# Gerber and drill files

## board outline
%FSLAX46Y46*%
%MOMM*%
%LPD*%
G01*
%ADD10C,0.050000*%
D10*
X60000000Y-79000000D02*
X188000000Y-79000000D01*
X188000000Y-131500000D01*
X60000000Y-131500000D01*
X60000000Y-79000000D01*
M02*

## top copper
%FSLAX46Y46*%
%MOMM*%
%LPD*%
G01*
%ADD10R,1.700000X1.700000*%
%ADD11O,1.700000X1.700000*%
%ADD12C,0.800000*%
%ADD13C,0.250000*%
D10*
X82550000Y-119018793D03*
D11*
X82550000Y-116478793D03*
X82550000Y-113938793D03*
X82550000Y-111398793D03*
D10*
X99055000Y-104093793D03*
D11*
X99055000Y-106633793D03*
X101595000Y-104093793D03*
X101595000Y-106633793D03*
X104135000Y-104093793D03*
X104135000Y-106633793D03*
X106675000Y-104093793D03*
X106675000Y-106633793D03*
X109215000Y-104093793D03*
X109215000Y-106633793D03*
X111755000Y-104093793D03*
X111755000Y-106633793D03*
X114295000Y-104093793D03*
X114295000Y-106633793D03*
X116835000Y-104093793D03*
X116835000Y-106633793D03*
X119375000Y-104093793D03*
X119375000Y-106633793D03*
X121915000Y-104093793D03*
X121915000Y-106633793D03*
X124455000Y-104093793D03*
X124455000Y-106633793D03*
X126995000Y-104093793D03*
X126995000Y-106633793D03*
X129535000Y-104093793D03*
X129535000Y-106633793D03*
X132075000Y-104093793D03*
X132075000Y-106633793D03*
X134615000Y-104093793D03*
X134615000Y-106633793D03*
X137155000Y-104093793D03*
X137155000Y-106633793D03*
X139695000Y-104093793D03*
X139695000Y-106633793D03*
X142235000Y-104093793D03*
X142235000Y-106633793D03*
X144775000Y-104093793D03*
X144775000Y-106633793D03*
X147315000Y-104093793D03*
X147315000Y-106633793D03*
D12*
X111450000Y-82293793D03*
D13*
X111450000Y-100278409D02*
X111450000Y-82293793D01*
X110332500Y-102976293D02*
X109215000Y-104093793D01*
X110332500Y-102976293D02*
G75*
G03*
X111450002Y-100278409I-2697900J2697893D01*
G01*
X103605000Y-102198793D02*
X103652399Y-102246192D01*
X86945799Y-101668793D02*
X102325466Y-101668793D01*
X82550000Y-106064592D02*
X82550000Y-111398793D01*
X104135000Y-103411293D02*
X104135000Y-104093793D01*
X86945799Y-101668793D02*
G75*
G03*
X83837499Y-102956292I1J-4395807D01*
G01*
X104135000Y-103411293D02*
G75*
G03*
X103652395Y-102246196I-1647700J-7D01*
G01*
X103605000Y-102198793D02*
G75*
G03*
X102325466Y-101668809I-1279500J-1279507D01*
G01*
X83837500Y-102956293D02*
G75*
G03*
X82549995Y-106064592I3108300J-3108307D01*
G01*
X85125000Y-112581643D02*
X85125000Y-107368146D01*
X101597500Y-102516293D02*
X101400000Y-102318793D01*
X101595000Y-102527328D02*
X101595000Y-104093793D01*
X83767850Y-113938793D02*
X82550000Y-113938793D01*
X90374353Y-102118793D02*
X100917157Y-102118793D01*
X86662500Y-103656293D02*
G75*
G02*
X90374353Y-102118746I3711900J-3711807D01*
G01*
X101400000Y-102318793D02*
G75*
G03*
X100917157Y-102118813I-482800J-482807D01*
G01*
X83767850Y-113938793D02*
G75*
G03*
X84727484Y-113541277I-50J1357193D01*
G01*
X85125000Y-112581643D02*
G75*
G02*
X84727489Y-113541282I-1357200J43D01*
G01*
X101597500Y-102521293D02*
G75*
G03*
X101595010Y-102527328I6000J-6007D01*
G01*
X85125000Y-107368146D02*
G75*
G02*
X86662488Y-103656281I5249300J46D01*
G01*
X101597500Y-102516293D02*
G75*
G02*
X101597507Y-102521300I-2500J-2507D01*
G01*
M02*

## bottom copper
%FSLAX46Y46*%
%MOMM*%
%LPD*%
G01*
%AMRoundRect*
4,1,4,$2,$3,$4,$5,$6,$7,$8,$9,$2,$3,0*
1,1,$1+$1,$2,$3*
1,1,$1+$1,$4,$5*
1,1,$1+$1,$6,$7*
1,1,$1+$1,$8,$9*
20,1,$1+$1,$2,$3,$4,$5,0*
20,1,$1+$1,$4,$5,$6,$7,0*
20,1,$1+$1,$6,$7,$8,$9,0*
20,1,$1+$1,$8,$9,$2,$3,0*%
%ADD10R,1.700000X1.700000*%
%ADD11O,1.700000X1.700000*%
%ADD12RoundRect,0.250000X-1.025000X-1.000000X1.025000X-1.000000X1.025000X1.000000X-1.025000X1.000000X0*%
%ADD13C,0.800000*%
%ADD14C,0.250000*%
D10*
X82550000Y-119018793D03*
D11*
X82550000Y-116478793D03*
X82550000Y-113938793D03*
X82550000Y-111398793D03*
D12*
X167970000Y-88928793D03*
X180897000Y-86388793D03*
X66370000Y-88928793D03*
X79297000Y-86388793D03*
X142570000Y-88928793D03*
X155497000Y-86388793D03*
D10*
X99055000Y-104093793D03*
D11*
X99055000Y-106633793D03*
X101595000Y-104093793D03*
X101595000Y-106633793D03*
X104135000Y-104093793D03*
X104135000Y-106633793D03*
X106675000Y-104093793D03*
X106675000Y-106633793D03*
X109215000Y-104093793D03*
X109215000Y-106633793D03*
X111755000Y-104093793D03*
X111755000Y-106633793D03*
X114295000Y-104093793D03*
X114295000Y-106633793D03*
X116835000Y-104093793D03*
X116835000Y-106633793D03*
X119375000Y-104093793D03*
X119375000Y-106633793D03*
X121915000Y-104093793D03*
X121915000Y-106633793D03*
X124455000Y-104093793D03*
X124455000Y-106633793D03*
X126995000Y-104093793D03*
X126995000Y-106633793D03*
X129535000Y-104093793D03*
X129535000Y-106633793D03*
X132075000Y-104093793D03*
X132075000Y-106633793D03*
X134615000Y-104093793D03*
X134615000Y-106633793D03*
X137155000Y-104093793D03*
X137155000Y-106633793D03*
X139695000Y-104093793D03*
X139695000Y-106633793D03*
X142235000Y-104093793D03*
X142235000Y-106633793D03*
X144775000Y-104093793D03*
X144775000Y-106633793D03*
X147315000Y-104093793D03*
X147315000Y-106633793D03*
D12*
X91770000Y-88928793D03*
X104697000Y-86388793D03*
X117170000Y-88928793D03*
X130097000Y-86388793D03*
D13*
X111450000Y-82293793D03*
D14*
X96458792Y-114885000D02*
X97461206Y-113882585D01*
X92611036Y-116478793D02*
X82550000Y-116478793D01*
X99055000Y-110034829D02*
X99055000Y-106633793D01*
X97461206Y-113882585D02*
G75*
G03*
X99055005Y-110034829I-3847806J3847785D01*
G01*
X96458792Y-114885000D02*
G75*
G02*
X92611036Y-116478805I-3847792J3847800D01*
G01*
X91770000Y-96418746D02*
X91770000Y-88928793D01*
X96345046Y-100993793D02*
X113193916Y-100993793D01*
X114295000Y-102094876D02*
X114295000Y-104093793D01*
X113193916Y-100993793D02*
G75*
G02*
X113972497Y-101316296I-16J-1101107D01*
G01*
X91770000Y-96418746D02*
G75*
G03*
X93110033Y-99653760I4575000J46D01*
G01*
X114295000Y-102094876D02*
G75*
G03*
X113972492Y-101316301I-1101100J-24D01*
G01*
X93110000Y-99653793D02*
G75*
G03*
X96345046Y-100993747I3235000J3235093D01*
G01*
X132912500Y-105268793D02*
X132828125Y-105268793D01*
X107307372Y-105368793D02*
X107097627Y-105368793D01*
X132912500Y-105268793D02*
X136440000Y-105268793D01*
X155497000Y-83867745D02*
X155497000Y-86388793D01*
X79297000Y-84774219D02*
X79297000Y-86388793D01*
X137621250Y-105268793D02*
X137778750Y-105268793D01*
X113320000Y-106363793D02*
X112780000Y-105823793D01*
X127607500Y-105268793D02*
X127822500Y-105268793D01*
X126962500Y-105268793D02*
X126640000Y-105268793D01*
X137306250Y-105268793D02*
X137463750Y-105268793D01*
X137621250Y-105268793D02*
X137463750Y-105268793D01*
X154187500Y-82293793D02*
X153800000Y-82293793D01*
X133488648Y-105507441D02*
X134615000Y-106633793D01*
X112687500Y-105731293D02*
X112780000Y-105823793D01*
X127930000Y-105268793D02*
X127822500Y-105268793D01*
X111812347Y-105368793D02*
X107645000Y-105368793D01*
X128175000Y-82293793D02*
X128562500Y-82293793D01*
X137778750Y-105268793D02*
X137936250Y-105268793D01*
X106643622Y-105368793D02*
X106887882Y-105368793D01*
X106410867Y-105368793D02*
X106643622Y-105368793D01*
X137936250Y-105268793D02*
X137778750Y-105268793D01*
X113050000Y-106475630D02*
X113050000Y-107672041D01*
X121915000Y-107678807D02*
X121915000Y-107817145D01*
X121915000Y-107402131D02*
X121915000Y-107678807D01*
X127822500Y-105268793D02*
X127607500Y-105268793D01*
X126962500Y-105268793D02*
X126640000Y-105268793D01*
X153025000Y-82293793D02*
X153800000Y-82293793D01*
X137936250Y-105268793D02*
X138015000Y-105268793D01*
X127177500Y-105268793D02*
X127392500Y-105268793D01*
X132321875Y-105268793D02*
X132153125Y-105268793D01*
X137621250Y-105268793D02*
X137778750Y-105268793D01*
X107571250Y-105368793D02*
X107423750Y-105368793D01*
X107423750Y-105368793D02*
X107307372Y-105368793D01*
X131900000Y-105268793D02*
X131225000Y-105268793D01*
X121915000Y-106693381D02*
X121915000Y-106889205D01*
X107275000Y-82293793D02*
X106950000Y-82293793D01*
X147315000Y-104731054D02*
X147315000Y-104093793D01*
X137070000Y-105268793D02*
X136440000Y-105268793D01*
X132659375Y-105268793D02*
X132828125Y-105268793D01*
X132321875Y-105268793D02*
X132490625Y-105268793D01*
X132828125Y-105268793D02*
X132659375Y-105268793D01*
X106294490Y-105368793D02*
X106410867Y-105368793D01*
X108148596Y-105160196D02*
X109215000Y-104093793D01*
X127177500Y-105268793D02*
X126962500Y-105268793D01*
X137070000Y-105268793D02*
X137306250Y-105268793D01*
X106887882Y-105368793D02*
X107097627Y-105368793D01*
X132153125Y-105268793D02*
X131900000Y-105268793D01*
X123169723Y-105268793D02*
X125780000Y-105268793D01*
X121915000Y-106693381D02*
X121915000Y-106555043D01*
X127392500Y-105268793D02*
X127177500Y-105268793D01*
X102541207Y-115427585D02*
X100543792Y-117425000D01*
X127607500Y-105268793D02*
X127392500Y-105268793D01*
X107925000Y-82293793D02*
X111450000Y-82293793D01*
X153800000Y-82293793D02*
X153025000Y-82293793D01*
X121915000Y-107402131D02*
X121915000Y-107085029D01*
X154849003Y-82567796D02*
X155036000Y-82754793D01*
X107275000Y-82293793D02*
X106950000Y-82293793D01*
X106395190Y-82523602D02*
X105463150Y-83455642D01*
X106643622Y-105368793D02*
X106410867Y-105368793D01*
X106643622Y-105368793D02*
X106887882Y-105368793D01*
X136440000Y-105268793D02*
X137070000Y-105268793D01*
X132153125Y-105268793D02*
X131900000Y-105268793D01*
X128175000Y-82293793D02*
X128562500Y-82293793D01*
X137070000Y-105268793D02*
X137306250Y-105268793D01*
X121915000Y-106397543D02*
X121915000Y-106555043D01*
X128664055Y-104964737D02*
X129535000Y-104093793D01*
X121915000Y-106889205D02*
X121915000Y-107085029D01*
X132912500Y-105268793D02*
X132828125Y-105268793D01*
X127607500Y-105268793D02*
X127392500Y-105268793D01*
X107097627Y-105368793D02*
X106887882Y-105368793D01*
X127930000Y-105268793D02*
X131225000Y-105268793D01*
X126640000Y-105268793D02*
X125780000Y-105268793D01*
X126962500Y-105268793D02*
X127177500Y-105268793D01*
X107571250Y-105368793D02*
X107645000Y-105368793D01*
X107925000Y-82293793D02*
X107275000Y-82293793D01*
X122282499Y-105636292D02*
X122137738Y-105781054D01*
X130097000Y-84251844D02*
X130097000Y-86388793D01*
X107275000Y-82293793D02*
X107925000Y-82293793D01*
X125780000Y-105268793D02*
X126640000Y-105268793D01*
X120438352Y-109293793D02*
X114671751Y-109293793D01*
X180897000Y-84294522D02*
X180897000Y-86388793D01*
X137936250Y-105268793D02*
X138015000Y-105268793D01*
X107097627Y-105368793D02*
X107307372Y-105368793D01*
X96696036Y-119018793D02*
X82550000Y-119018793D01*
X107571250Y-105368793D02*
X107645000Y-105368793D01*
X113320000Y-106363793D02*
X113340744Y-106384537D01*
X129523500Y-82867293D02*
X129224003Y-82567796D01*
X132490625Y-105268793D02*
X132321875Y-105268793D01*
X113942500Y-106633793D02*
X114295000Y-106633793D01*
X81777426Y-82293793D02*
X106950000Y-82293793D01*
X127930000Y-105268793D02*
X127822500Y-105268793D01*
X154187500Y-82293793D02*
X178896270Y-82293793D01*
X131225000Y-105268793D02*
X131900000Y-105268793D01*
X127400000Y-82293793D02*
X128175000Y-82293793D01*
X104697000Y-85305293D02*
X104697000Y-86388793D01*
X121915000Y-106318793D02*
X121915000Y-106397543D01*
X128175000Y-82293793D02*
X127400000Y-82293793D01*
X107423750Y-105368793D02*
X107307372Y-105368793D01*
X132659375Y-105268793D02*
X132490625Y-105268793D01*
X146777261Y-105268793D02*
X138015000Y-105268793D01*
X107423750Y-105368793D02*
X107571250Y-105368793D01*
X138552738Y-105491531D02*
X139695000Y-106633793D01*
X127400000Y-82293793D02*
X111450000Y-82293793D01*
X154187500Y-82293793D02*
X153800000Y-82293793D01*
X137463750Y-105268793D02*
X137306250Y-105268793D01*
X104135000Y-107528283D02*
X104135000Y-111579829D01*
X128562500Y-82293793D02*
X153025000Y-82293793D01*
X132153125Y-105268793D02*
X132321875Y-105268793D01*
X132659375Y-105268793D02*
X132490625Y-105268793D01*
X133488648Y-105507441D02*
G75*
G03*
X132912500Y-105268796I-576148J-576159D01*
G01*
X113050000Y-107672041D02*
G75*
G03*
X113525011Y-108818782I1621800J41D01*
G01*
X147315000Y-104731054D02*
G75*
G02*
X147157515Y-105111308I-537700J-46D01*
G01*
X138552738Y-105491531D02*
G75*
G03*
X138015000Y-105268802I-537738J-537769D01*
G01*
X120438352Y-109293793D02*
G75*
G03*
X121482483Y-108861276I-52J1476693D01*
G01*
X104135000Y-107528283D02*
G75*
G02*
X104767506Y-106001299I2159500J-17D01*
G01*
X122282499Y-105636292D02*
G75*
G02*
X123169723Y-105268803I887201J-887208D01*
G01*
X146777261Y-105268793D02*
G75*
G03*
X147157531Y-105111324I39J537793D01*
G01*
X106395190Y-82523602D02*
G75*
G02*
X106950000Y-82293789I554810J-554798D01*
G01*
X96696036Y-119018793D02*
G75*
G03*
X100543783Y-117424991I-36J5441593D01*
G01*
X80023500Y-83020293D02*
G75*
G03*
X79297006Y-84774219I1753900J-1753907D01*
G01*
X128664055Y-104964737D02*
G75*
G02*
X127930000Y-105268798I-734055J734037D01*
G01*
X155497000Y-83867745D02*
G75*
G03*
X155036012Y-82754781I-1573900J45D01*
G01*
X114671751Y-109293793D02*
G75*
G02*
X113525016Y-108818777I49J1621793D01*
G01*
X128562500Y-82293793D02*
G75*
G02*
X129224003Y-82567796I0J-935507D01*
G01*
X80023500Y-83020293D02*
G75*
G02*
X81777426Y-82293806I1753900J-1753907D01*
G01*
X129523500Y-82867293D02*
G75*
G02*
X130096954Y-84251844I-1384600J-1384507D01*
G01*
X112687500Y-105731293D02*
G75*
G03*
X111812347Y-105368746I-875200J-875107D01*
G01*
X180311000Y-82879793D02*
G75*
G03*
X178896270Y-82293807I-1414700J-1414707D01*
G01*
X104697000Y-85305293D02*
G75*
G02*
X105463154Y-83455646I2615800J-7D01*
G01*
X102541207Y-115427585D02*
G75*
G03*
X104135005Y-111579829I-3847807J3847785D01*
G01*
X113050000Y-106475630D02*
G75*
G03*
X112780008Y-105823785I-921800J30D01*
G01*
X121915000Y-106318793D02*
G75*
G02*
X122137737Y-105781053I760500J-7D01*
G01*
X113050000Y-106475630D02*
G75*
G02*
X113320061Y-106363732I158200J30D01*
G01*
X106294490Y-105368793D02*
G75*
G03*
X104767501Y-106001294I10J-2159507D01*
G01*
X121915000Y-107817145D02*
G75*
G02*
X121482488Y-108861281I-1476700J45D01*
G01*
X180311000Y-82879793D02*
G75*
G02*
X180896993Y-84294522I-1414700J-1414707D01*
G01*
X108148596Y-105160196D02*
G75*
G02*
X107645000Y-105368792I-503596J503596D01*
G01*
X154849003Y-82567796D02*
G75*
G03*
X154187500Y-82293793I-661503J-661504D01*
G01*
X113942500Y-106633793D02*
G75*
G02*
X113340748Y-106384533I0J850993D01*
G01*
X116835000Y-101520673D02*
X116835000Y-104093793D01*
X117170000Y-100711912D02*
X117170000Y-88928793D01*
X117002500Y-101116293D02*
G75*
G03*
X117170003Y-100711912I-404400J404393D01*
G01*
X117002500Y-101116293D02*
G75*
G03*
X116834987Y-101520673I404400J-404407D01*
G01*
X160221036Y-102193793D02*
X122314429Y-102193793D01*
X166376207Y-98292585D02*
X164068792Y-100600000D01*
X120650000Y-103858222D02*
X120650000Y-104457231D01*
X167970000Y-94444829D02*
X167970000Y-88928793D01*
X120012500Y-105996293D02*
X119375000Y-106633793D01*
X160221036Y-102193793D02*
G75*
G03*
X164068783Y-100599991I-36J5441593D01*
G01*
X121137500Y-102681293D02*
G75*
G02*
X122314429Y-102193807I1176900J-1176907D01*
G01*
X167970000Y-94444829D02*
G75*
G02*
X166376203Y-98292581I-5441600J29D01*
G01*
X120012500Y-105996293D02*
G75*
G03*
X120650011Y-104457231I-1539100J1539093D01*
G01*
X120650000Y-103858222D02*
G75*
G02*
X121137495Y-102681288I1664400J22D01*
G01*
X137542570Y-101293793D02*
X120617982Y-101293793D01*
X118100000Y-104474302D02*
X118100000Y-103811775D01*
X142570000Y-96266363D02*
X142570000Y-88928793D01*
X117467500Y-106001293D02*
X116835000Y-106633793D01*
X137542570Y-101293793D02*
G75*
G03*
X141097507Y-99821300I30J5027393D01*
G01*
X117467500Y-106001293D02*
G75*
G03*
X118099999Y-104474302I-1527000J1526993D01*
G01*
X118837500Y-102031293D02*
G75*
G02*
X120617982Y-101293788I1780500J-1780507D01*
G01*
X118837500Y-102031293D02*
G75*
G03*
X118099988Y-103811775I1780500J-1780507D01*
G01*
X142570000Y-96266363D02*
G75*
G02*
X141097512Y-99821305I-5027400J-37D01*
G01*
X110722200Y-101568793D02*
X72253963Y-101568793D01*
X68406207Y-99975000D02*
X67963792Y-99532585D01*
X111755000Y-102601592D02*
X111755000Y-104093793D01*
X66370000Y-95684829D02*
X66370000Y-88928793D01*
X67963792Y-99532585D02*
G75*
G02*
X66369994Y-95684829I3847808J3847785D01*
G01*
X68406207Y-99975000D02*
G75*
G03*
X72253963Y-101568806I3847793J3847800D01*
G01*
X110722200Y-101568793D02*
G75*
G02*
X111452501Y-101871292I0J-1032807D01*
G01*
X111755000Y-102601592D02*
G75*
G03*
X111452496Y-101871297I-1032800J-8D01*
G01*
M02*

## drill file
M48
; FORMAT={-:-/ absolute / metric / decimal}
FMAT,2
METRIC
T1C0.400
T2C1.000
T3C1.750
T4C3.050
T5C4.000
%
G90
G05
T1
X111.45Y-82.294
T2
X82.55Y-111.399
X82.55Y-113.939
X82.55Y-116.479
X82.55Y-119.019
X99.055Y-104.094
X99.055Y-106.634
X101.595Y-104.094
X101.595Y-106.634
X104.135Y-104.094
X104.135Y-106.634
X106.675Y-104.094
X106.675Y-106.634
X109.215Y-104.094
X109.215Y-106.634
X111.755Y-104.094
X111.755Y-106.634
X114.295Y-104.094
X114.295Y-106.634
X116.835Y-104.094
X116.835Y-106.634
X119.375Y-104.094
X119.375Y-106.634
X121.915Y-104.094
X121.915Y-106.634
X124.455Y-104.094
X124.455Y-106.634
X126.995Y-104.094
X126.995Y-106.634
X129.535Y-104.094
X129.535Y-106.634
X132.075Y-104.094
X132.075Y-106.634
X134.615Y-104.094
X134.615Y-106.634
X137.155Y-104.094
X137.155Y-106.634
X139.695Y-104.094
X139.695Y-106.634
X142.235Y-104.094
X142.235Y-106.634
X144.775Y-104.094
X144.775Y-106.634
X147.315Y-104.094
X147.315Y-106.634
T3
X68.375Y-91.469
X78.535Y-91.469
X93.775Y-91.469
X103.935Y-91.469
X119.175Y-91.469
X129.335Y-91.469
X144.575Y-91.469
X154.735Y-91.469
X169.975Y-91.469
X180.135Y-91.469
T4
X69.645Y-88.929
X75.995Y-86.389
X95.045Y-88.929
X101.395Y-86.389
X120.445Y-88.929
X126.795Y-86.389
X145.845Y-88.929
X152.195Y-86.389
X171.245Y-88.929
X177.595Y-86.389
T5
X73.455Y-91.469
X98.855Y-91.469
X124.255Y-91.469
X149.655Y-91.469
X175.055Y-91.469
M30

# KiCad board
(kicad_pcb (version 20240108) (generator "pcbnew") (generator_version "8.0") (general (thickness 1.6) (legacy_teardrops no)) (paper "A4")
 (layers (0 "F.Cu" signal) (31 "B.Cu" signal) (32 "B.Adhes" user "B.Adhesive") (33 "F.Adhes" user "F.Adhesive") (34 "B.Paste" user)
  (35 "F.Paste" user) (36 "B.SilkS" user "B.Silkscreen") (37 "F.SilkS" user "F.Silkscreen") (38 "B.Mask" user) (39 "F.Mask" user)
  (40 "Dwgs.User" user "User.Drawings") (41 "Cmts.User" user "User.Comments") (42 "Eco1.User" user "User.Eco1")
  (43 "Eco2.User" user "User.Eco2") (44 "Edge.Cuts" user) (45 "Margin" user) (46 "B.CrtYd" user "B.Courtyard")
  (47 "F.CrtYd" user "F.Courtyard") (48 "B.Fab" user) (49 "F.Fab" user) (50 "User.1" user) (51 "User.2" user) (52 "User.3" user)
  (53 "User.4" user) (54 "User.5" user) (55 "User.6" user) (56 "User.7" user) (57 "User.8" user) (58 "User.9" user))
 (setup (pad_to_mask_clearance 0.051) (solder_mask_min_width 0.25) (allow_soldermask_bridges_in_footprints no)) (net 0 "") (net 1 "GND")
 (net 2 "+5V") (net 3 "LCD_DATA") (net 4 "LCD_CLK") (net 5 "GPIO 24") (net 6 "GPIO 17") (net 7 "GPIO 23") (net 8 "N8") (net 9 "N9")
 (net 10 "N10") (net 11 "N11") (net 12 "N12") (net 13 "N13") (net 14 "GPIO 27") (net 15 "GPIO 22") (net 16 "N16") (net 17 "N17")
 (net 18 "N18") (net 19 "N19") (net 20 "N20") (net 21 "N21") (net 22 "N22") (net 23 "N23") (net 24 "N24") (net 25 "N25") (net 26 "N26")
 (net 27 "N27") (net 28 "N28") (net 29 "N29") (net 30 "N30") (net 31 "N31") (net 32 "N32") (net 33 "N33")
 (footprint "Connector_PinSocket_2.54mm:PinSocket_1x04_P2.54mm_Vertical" (layer "F.Cu") (at 82.55 119.018793 180)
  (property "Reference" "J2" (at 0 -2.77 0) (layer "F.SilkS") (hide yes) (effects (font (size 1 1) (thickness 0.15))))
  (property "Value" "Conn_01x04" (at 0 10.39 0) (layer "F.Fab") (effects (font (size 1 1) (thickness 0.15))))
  (pad "1" thru_hole rect (at 0 0 180) (size 1.7 1.7) (drill 1) (layers "*.Cu" "*.Mask") (remove_unused_layers no) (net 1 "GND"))
  (pad "2" thru_hole oval (at 0 2.54 180) (size 1.7 1.7) (drill 1) (layers "*.Cu" "*.Mask") (remove_unused_layers no) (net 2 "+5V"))
  (pad "3" thru_hole oval (at 0 5.08 180) (size 1.7 1.7) (drill 1) (layers "*.Cu" "*.Mask") (remove_unused_layers no) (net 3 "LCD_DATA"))
  (pad "4" thru_hole oval (at 0 7.62 180) (size 1.7 1.7) (drill 1) (layers "*.Cu" "*.Mask") (remove_unused_layers no) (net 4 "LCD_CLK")))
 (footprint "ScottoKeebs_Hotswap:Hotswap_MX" (layer "F.Cu") (at 175.055 91.468793)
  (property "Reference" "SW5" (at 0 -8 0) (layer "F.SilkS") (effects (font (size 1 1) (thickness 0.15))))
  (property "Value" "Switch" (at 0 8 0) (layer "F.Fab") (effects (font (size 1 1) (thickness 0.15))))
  (pad "" np_thru_hole circle (at -5.08 0) (size 1.75 1.75) (drill 1.75) (layers "*.Cu" "*.Mask"))
  (pad "" np_thru_hole circle (at -3.81 -2.54) (size 3.05 3.05) (drill 3.05) (layers "*.Cu" "*.Mask"))
  (pad "" np_thru_hole circle (at 0 0) (size 4 4) (drill 4) (layers "*.Cu" "*.Mask"))
  (pad "" np_thru_hole circle (at 2.54 -5.08) (size 3.05 3.05) (drill 3.05) (layers "*.Cu" "*.Mask"))
  (pad "" np_thru_hole circle (at 5.08 0) (size 1.75 1.75) (drill 1.75) (layers "*.Cu" "*.Mask"))
  (pad "1" smd roundrect (at -7.085 -2.54) (size 2.55 2.5) (layers "B.Cu" "B.Paste" "B.Mask") (roundrect_rratio 0.1) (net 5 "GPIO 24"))
  (pad "2" smd roundrect (at 5.842 -5.08) (size 2.55 2.5) (layers "B.Cu" "B.Paste" "B.Mask") (roundrect_rratio 0.1) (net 1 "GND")))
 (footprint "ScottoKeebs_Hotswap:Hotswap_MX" (layer "F.Cu") (at 73.455 91.468793)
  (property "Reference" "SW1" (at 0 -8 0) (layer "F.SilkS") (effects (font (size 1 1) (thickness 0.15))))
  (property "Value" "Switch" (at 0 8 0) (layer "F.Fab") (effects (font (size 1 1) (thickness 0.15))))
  (pad "" np_thru_hole circle (at -5.08 0) (size 1.75 1.75) (drill 1.75) (layers "*.Cu" "*.Mask"))
  (pad "" np_thru_hole circle (at -3.81 -2.54) (size 3.05 3.05) (drill 3.05) (layers "*.Cu" "*.Mask"))
  (pad "" np_thru_hole circle (at 0 0) (size 4 4) (drill 4) (layers "*.Cu" "*.Mask"))
  (pad "" np_thru_hole circle (at 2.54 -5.08) (size 3.05 3.05) (drill 3.05) (layers "*.Cu" "*.Mask"))
  (pad "" np_thru_hole circle (at 5.08 0) (size 1.75 1.75) (drill 1.75) (layers "*.Cu" "*.Mask"))
  (pad "1" smd roundrect (at -7.085 -2.54) (size 2.55 2.5) (layers "B.Cu" "B.Paste" "B.Mask") (roundrect_rratio 0.1) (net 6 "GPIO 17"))
  (pad "2" smd roundrect (at 5.842 -5.08) (size 2.55 2.5) (layers "B.Cu" "B.Paste" "B.Mask") (roundrect_rratio 0.1) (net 1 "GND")))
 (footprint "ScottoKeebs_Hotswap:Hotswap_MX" (layer "F.Cu") (at 149.655 91.468793)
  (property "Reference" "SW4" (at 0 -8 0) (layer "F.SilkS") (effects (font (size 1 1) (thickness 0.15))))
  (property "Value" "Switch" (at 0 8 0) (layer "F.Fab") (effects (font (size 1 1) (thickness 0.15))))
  (pad "" np_thru_hole circle (at -5.08 0) (size 1.75 1.75) (drill 1.75) (layers "*.Cu" "*.Mask"))
  (pad "" np_thru_hole circle (at -3.81 -2.54) (size 3.05 3.05) (drill 3.05) (layers "*.Cu" "*.Mask"))
  (pad "" np_thru_hole circle (at 0 0) (size 4 4) (drill 4) (layers "*.Cu" "*.Mask"))
  (pad "" np_thru_hole circle (at 2.54 -5.08) (size 3.05 3.05) (drill 3.05) (layers "*.Cu" "*.Mask"))
  (pad "" np_thru_hole circle (at 5.08 0) (size 1.75 1.75) (drill 1.75) (layers "*.Cu" "*.Mask"))
  (pad "1" smd roundrect (at -7.085 -2.54) (size 2.55 2.5) (layers "B.Cu" "B.Paste" "B.Mask") (roundrect_rratio 0.1) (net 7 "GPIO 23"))
  (pad "2" smd roundrect (at 5.842 -5.08) (size 2.55 2.5) (layers "B.Cu" "B.Paste" "B.Mask") (roundrect_rratio 0.1) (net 1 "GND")))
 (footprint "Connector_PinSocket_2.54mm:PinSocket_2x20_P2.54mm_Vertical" (layer "F.Cu") (at 99.055 104.093793 90)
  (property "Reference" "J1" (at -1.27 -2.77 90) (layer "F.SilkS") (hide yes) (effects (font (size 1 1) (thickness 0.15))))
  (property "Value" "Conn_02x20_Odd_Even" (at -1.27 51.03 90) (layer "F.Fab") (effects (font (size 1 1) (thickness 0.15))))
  (pad "1" thru_hole rect (at 0 0 90) (size 1.7 1.7) (drill 1) (layers "*.Cu" "*.Mask") (remove_unused_layers no) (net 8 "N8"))
  (pad "2" thru_hole oval (at -2.54 0 90) (size 1.7 1.7) (drill 1) (layers "*.Cu" "*.Mask") (remove_unused_layers no) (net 2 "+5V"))
  (pad "3" thru_hole oval (at 0 2.54 90) (size 1.7 1.7) (drill 1) (layers "*.Cu" "*.Mask") (remove_unused_layers no) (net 3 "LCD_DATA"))
  (pad "4" thru_hole oval (at -2.54 2.54 90) (size 1.7 1.7) (drill 1) (layers "*.Cu" "*.Mask") (remove_unused_layers no) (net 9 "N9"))
  (pad "5" thru_hole oval (at 0 5.08 90) (size 1.7 1.7) (drill 1) (layers "*.Cu" "*.Mask") (remove_unused_layers no) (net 4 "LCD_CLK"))
  (pad "6" thru_hole oval (at -2.54 5.08 90) (size 1.7 1.7) (drill 1) (layers "*.Cu" "*.Mask") (remove_unused_layers no) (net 1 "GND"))
  (pad "7" thru_hole oval (at 0 7.62 90) (size 1.7 1.7) (drill 1) (layers "*.Cu" "*.Mask") (remove_unused_layers no) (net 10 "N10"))
  (pad "8" thru_hole oval (at -2.54 7.62 90) (size 1.7 1.7) (drill 1) (layers "*.Cu" "*.Mask") (remove_unused_layers no) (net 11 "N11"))
  (pad "9" thru_hole oval (at 0 10.16 90) (size 1.7 1.7) (drill 1) (layers "*.Cu" "*.Mask") (remove_unused_layers no) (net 1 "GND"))
  (pad "10" thru_hole oval (at -2.54 10.16 90) (size 1.7 1.7) (drill 1) (layers "*.Cu" "*.Mask") (remove_unused_layers no) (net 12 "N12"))
  (pad "11" thru_hole oval (at 0 12.7 90) (size 1.7 1.7) (drill 1) (layers "*.Cu" "*.Mask") (remove_unused_layers no) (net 6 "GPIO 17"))
  (pad "12" thru_hole oval (at -2.54 12.7 90) (size 1.7 1.7) (drill 1) (layers "*.Cu" "*.Mask") (remove_unused_layers no) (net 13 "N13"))
  (pad "13" thru_hole oval (at 0 15.24 90) (size 1.7 1.7) (drill 1) (layers "*.Cu" "*.Mask") (remove_unused_layers no) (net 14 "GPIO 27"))
  (pad "14" thru_hole oval (at -2.54 15.24 90) (size 1.7 1.7) (drill 1) (layers "*.Cu" "*.Mask") (remove_unused_layers no) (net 1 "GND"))
  (pad "15" thru_hole oval (at 0 17.78 90) (size 1.7 1.7) (drill 1) (layers "*.Cu" "*.Mask") (remove_unused_layers no) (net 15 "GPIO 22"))
  (pad "16" thru_hole oval (at -2.54 17.78 90) (size 1.7 1.7) (drill 1) (layers "*.Cu" "*.Mask") (remove_unused_layers no) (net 7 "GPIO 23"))
  (pad "17" thru_hole oval (at 0 20.32 90) (size 1.7 1.7) (drill 1) (layers "*.Cu" "*.Mask") (remove_unused_layers no) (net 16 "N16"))
  (pad "18" thru_hole oval (at -2.54 20.32 90) (size 1.7 1.7) (drill 1) (layers "*.Cu" "*.Mask") (remove_unused_layers no) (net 5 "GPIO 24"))
  (pad "19" thru_hole oval (at 0 22.86 90) (size 1.7 1.7) (drill 1) (layers "*.Cu" "*.Mask") (remove_unused_layers no) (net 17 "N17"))
  (pad "20" thru_hole oval (at -2.54 22.86 90) (size 1.7 1.7) (drill 1) (layers "*.Cu" "*.Mask") (remove_unused_layers no) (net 1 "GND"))
  (pad "21" thru_hole oval (at 0 25.4 90) (size 1.7 1.7) (drill 1) (layers "*.Cu" "*.Mask") (remove_unused_layers no) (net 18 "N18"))
  (pad "22" thru_hole oval (at -2.54 25.4 90) (size 1.7 1.7) (drill 1) (layers "*.Cu" "*.Mask") (remove_unused_layers no) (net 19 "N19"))
  (pad "23" thru_hole oval (at 0 27.94 90) (size 1.7 1.7) (drill 1) (layers "*.Cu" "*.Mask") (remove_unused_layers no) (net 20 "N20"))
  (pad "24" thru_hole oval (at -2.54 27.94 90) (size 1.7 1.7) (drill 1) (layers "*.Cu" "*.Mask") (remove_unused_layers no) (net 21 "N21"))
  (pad "25" thru_hole oval (at 0 30.48 90) (size 1.7 1.7) (drill 1) (layers "*.Cu" "*.Mask") (remove_unused_layers no) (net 1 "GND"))
  (pad "26" thru_hole oval (at -2.54 30.48 90) (size 1.7 1.7) (drill 1) (layers "*.Cu" "*.Mask") (remove_unused_layers no) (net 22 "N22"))
  (pad "27" thru_hole oval (at 0 33.02 90) (size 1.7 1.7) (drill 1) (layers "*.Cu" "*.Mask") (remove_unused_layers no) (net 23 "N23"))
  (pad "28" thru_hole oval (at -2.54 33.02 90) (size 1.7 1.7) (drill 1) (layers "*.Cu" "*.Mask") (remove_unused_layers no) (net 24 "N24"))
  (pad "29" thru_hole oval (at 0 35.56 90) (size 1.7 1.7) (drill 1) (layers "*.Cu" "*.Mask") (remove_unused_layers no) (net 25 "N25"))
  (pad "30" thru_hole oval (at -2.54 35.56 90) (size 1.7 1.7) (drill 1) (layers "*.Cu" "*.Mask") (remove_unused_layers no) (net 1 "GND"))
  (pad "31" thru_hole oval (at 0 38.1 90) (size 1.7 1.7) (drill 1) (layers "*.Cu" "*.Mask") (remove_unused_layers no) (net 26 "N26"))
  (pad "32" thru_hole oval (at -2.54 38.1 90) (size 1.7 1.7) (drill 1) (layers "*.Cu" "*.Mask") (remove_unused_layers no) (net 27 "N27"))
  (pad "33" thru_hole oval (at 0 40.64 90) (size 1.7 1.7) (drill 1) (layers "*.Cu" "*.Mask") (remove_unused_layers no) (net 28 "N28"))
  (pad "34" thru_hole oval (at -2.54 40.64 90) (size 1.7 1.7) (drill 1) (layers "*.Cu" "*.Mask") (remove_unused_layers no) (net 1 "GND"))
  (pad "35" thru_hole oval (at 0 43.18 90) (size 1.7 1.7) (drill 1) (layers "*.Cu" "*.Mask") (remove_unused_layers no) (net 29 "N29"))
  (pad "36" thru_hole oval (at -2.54 43.18 90) (size 1.7 1.7) (drill 1) (layers "*.Cu" "*.Mask") (remove_unused_layers no) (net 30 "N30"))
  (pad "37" thru_hole oval (at 0 45.72 90) (size 1.7 1.7) (drill 1) (layers "*.Cu" "*.Mask") (remove_unused_layers no) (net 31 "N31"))
  (pad "38" thru_hole oval (at -2.54 45.72 90) (size 1.7 1.7) (drill 1) (layers "*.Cu" "*.Mask") (remove_unused_layers no) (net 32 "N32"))
  (pad "39" thru_hole oval (at 0 48.26 90) (size 1.7 1.7) (drill 1) (layers "*.Cu" "*.Mask") (remove_unused_layers no) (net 1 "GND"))
  (pad "40" thru_hole oval (at -2.54 48.26 90) (size 1.7 1.7) (drill 1) (layers "*.Cu" "*.Mask") (remove_unused_layers no) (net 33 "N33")))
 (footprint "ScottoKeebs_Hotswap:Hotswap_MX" (layer "F.Cu") (at 98.855 91.468793)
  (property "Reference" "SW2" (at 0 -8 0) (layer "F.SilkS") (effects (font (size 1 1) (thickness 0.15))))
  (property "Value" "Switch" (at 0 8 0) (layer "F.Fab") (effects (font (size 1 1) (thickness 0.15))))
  (pad "" np_thru_hole circle (at -5.08 0) (size 1.75 1.75) (drill 1.75) (layers "*.Cu" "*.Mask"))
  (pad "" np_thru_hole circle (at -3.81 -2.54) (size 3.05 3.05) (drill 3.05) (layers "*.Cu" "*.Mask"))
  (pad "" np_thru_hole circle (at 0 0) (size 4 4) (drill 4) (layers "*.Cu" "*.Mask"))
  (pad "" np_thru_hole circle (at 2.54 -5.08) (size 3.05 3.05) (drill 3.05) (layers "*.Cu" "*.Mask"))
  (pad "" np_thru_hole circle (at 5.08 0) (size 1.75 1.75) (drill 1.75) (layers "*.Cu" "*.Mask"))
  (pad "1" smd roundrect (at -7.085 -2.54) (size 2.55 2.5) (layers "B.Cu" "B.Paste" "B.Mask") (roundrect_rratio 0.1) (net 14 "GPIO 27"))
  (pad "2" smd roundrect (at 5.842 -5.08) (size 2.55 2.5) (layers "B.Cu" "B.Paste" "B.Mask") (roundrect_rratio 0.1) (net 1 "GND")))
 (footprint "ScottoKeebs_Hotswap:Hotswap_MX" (layer "F.Cu") (at 124.255 91.468793)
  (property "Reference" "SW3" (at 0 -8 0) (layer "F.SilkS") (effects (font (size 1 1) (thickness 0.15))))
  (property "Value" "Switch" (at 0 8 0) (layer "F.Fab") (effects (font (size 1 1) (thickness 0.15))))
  (pad "" np_thru_hole circle (at -5.08 0) (size 1.75 1.75) (drill 1.75) (layers "*.Cu" "*.Mask"))
  (pad "" np_thru_hole circle (at -3.81 -2.54) (size 3.05 3.05) (drill 3.05) (layers "*.Cu" "*.Mask"))
  (pad "" np_thru_hole circle (at 0 0) (size 4 4) (drill 4) (layers "*.Cu" "*.Mask"))
  (pad "" np_thru_hole circle (at 2.54 -5.08) (size 3.05 3.05) (drill 3.05) (layers "*.Cu" "*.Mask"))
  (pad "" np_thru_hole circle (at 5.08 0) (size 1.75 1.75) (drill 1.75) (layers "*.Cu" "*.Mask"))
  (pad "1" smd roundrect (at -7.085 -2.54) (size 2.55 2.5) (layers "B.Cu" "B.Paste" "B.Mask") (roundrect_rratio 0.1) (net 15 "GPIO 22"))
  (pad "2" smd roundrect (at 5.842 -5.08) (size 2.55 2.5) (layers "B.Cu" "B.Paste" "B.Mask") (roundrect_rratio 0.1) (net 1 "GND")))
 (gr_rect (start 60 79) (end 188 131.5) (stroke (width 0.05) (type default)) (fill none) (layer "Edge.Cuts"))
 (segment (start 96.458792 114.885) (end 97.461206 113.882585) (width 0.25) (layer "B.Cu") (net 2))
 (segment (start 92.611036 116.478793) (end 82.55 116.478793) (width 0.25) (layer "B.Cu") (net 2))
 (segment (start 99.055 110.034829) (end 99.055 106.633793) (width 0.25) (layer "B.Cu") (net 2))
 (arc (start 97.461206 113.882585) (mid 98.640786 112.117219) (end 99.055 110.034829) (width 0.25) (layer "B.Cu") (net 2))
 (arc (start 96.458792 114.885) (mid 94.693426 116.064579) (end 92.611036 116.478793) (width 0.25) (layer "B.Cu") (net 2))
 (segment (start 91.77 96.418746) (end 91.77 88.928793) (width 0.25) (layer "B.Cu") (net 14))
 (segment (start 96.345046 100.993793) (end 113.193916 100.993793) (width 0.25) (layer "B.Cu") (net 14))
 (segment (start 114.295 102.094876) (end 114.295 104.093793) (width 0.25) (layer "B.Cu") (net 14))
 (arc (start 113.193916 100.993793) (mid 113.615282 101.077608) (end 113.9725 101.316293) (width 0.25) (layer "B.Cu") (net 14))
 (arc (start 91.77 96.418746) (mid 92.118254 98.16954) (end 93.11 99.653793) (width 0.25) (layer "B.Cu") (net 14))
 (arc (start 114.295 102.094876) (mid 114.211184 101.67351) (end 113.9725 101.316293) (width 0.25) (layer "B.Cu") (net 14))
 (arc (start 93.11 99.653793) (mid 94.594251 100.645538) (end 96.345046 100.993793) (width 0.25) (layer "B.Cu") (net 14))
 (segment (start 111.45 100.278409) (end 111.45 82.293793) (width 0.25) (layer "F.Cu") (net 1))
 (segment (start 110.3325 102.976293) (end 109.215 104.093793) (width 0.25) (layer "F.Cu") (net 1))
 (via (at 111.45 82.293793) (size 0.8) (drill 0.4) (layers "F.Cu" "B.Cu") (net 1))
 (arc (start 110.3325 102.976293) (mid 111.159571 101.738493) (end 111.45 100.278409) (width 0.25) (layer "F.Cu") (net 1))
 (segment (start 132.9125 105.268793) (end 132.828125 105.268793) (width 0.25) (layer "B.Cu") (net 1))
 (segment (start 107.307372 105.368793) (end 107.097627 105.368793) (width 0.25) (layer "B.Cu") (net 1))
 (segment (start 132.9125 105.268793) (end 136.44 105.268793) (width 0.25) (layer "B.Cu") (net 1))
 (segment (start 155.497 83.867745) (end 155.497 86.388793) (width 0.25) (layer "B.Cu") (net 1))
 (segment (start 79.297 84.774219) (end 79.297 86.388793) (width 0.25) (layer "B.Cu") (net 1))
 (segment (start 137.62125 105.268793) (end 137.77875 105.268793) (width 0.25) (layer "B.Cu") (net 1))
 (segment (start 113.32 106.363793) (end 112.78 105.823793) (width 0.25) (layer "B.Cu") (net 1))
 (segment (start 127.6075 105.268793) (end 127.8225 105.268793) (width 0.25) (layer "B.Cu") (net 1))
 (segment (start 126.9625 105.268793) (end 126.64 105.268793) (width 0.25) (layer "B.Cu") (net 1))
 (segment (start 137.30625 105.268793) (end 137.46375 105.268793) (width 0.25) (layer "B.Cu") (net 1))
 (segment (start 137.62125 105.268793) (end 137.46375 105.268793) (width 0.25) (layer "B.Cu") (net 1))
 (segment (start 154.1875 82.293793) (end 153.8 82.293793) (width 0.25) (layer "B.Cu") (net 1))
 (segment (start 133.488648 105.507441) (end 134.615 106.633793) (width 0.25) (layer "B.Cu") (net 1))
 (segment (start 112.6875 105.731293) (end 112.78 105.823793) (width 0.25) (layer "B.Cu") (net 1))
 (segment (start 127.93 105.268793) (end 127.8225 105.268793) (width 0.25) (layer "B.Cu") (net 1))
 (segment (start 111.812347 105.368793) (end 107.645 105.368793) (width 0.25) (layer "B.Cu") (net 1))
 (segment (start 128.175 82.293793) (end 128.5625 82.293793) (width 0.25) (layer "B.Cu") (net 1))
 (segment (start 137.77875 105.268793) (end 137.93625 105.268793) (width 0.25) (layer "B.Cu") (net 1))
 (segment (start 106.643622 105.368793) (end 106.887882 105.368793) (width 0.25) (layer "B.Cu") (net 1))
 (segment (start 106.410867 105.368793) (end 106.643622 105.368793) (width 0.25) (layer "B.Cu") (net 1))
 (segment (start 137.93625 105.268793) (end 137.77875 105.268793) (width 0.25) (layer "B.Cu") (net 1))
 (segment (start 113.05 106.47563) (end 113.05 107.672041) (width 0.25) (layer "B.Cu") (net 1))
 (segment (start 121.915 107.678807) (end 121.915 107.817145) (width 0.25) (layer "B.Cu") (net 1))
 (segment (start 121.915 107.402131) (end 121.915 107.678807) (width 0.25) (layer "B.Cu") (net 1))
 (segment (start 127.8225 105.268793) (end 127.6075 105.268793) (width 0.25) (layer "B.Cu") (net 1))
 (segment (start 126.9625 105.268793) (end 126.64 105.268793) (width 0.25) (layer "B.Cu") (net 1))
 (segment (start 153.025 82.293793) (end 153.8 82.293793) (width 0.25) (layer "B.Cu") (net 1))
 (segment (start 137.93625 105.268793) (end 138.015 105.268793) (width 0.25) (layer "B.Cu") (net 1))
 (segment (start 127.1775 105.268793) (end 127.3925 105.268793) (width 0.25) (layer "B.Cu") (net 1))
 (segment (start 132.321875 105.268793) (end 132.153125 105.268793) (width 0.25) (layer "B.Cu") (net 1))
 (segment (start 137.62125 105.268793) (end 137.77875 105.268793) (width 0.25) (layer "B.Cu") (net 1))
 (segment (start 107.57125 105.368793) (end 107.42375 105.368793) (width 0.25) (layer "B.Cu") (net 1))
 (segment (start 107.42375 105.368793) (end 107.307372 105.368793) (width 0.25) (layer "B.Cu") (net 1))
 (segment (start 131.9 105.268793) (end 131.225 105.268793) (width 0.25) (layer "B.Cu") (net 1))
 (segment (start 121.915 106.693381) (end 121.915 106.889205) (width 0.25) (layer "B.Cu") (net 1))
 (segment (start 107.275 82.293793) (end 106.95 82.293793) (width 0.25) (layer "B.Cu") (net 1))
 (segment (start 147.315 104.731054) (end 147.315 104.093793) (width 0.25) (layer "B.Cu") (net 1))
 (segment (start 137.07 105.268793) (end 136.44 105.268793) (width 0.25) (layer "B.Cu") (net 1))
 (segment (start 132.659375 105.268793) (end 132.828125 105.268793) (width 0.25) (layer "B.Cu") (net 1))
 (segment (start 132.321875 105.268793) (end 132.490625 105.268793) (width 0.25) (layer "B.Cu") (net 1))
 (segment (start 132.828125 105.268793) (end 132.659375 105.268793) (width 0.25) (layer "B.Cu") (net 1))
 (segment (start 106.29449 105.368793) (end 106.410867 105.368793) (width 0.25) (layer "B.Cu") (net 1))
 (segment (start 108.148596 105.160196) (end 109.215 104.093793) (width 0.25) (layer "B.Cu") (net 1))
 (segment (start 127.1775 105.268793) (end 126.9625 105.268793) (width 0.25) (layer "B.Cu") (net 1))
 (segment (start 137.07 105.268793) (end 137.30625 105.268793) (width 0.25) (layer "B.Cu") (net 1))
 (segment (start 106.887882 105.368793) (end 107.097627 105.368793) (width 0.25) (layer "B.Cu") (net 1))
 (segment (start 132.153125 105.268793) (end 131.9 105.268793) (width 0.25) (layer "B.Cu") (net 1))
 (segment (start 123.169723 105.268793) (end 125.78 105.268793) (width 0.25) (layer "B.Cu") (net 1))
 (segment (start 121.915 106.693381) (end 121.915 106.555043) (width 0.25) (layer "B.Cu") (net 1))
 (segment (start 127.3925 105.268793) (end 127.1775 105.268793) (width 0.25) (layer "B.Cu") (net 1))
 (segment (start 102.541207 115.427585) (end 100.543792 117.425) (width 0.25) (layer "B.Cu") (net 1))
 (segment (start 127.6075 105.268793) (end 127.3925 105.268793) (width 0.25) (layer "B.Cu") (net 1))
 (segment (start 107.925 82.293793) (end 111.45 82.293793) (width 0.25) (layer "B.Cu") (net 1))
 (segment (start 153.8 82.293793) (end 153.025 82.293793) (width 0.25) (layer "B.Cu") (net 1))
 (segment (start 121.915 107.402131) (end 121.915 107.085029) (width 0.25) (layer "B.Cu") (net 1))
 (segment (start 154.849003 82.567796) (end 155.036 82.754793) (width 0.25) (layer "B.Cu") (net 1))
 (segment (start 107.275 82.293793) (end 106.95 82.293793) (width 0.25) (layer "B.Cu") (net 1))
 (segment (start 106.39519 82.523602) (end 105.46315 83.455642) (width 0.25) (layer "B.Cu") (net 1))
 (segment (start 106.643622 105.368793) (end 106.410867 105.368793) (width 0.25) (layer "B.Cu") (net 1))
 (segment (start 106.643622 105.368793) (end 106.887882 105.368793) (width 0.25) (layer "B.Cu") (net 1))
 (segment (start 136.44 105.268793) (end 137.07 105.268793) (width 0.25) (layer "B.Cu") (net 1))
 (segment (start 132.153125 105.268793) (end 131.9 105.268793) (width 0.25) (layer "B.Cu") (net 1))
 (segment (start 128.175 82.293793) (end 128.5625 82.293793) (width 0.25) (layer "B.Cu") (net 1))
 (segment (start 137.07 105.268793) (end 137.30625 105.268793) (width 0.25) (layer "B.Cu") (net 1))
 (segment (start 121.915 106.397543) (end 121.915 106.555043) (width 0.25) (layer "B.Cu") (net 1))
 (segment (start 128.664055 104.964737) (end 129.535 104.093793) (width 0.25) (layer "B.Cu") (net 1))
 (segment (start 121.915 106.889205) (end 121.915 107.085029) (width 0.25) (layer "B.Cu") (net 1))
 (segment (start 132.9125 105.268793) (end 132.828125 105.268793) (width 0.25) (layer "B.Cu") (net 1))
 (segment (start 127.6075 105.268793) (end 127.3925 105.268793) (width 0.25) (layer "B.Cu") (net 1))
 (segment (start 107.097627 105.368793) (end 106.887882 105.368793) (width 0.25) (layer "B.Cu") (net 1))
 (segment (start 127.93 105.268793) (end 131.225 105.268793) (width 0.25) (layer "B.Cu") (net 1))
 (segment (start 126.64 105.268793) (end 125.78 105.268793) (width 0.25) (layer "B.Cu") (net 1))
 (segment (start 126.9625 105.268793) (end 127.1775 105.268793) (width 0.25) (layer "B.Cu") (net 1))
 (segment (start 107.57125 105.368793) (end 107.645 105.368793) (width 0.25) (layer "B.Cu") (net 1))
 (segment (start 107.925 82.293793) (end 107.275 82.293793) (width 0.25) (layer "B.Cu") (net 1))
 (segment (start 122.282499 105.636292) (end 122.137738 105.781054) (width 0.25) (layer "B.Cu") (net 1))
 (segment (start 130.097 84.251844) (end 130.097 86.388793) (width 0.25) (layer "B.Cu") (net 1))
 (segment (start 107.275 82.293793) (end 107.925 82.293793) (width 0.25) (layer "B.Cu") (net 1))
 (segment (start 125.78 105.268793) (end 126.64 105.268793) (width 0.25) (layer "B.Cu") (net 1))
 (segment (start 120.438352 109.293793) (end 114.671751 109.293793) (width 0.25) (layer "B.Cu") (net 1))
 (segment (start 180.897 84.294522) (end 180.897 86.388793) (width 0.25) (layer "B.Cu") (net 1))
 (segment (start 137.93625 105.268793) (end 138.015 105.268793) (width 0.25) (layer "B.Cu") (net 1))
 (segment (start 107.097627 105.368793) (end 107.307372 105.368793) (width 0.25) (layer "B.Cu") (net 1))
 (segment (start 96.696036 119.018793) (end 82.55 119.018793) (width 0.25) (layer "B.Cu") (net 1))
 (segment (start 107.57125 105.368793) (end 107.645 105.368793) (width 0.25) (layer "B.Cu") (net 1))
 (segment (start 113.32 106.363793) (end 113.340744 106.384537) (width 0.25) (layer "B.Cu") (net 1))
 (segment (start 129.5235 82.867293) (end 129.224003 82.567796) (width 0.25) (layer "B.Cu") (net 1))
 (segment (start 132.490625 105.268793) (end 132.321875 105.268793) (width 0.25) (layer "B.Cu") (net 1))
 (segment (start 113.9425 106.633793) (end 114.295 106.633793) (width 0.25) (layer "B.Cu") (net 1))
 (segment (start 81.777426 82.293793) (end 106.95 82.293793) (width 0.25) (layer "B.Cu") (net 1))
 (segment (start 127.93 105.268793) (end 127.8225 105.268793) (width 0.25) (layer "B.Cu") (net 1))
 (segment (start 154.1875 82.293793) (end 178.89627 82.293793) (width 0.25) (layer "B.Cu") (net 1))
 (segment (start 131.225 105.268793) (end 131.9 105.268793) (width 0.25) (layer "B.Cu") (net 1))
 (segment (start 127.4 82.293793) (end 128.175 82.293793) (width 0.25) (layer "B.Cu") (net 1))
 (segment (start 104.697 85.305293) (end 104.697 86.388793) (width 0.25) (layer "B.Cu") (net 1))
 (segment (start 121.915 106.318793) (end 121.915 106.397543) (width 0.25) (layer "B.Cu") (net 1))
 (segment (start 128.175 82.293793) (end 127.4 82.293793) (width 0.25) (layer "B.Cu") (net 1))
 (segment (start 107.42375 105.368793) (end 107.307372 105.368793) (width 0.25) (layer "B.Cu") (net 1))
 (segment (start 132.659375 105.268793) (end 132.490625 105.268793) (width 0.25) (layer "B.Cu") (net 1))
 (segment (start 146.777261 105.268793) (end 138.015 105.268793) (width 0.25) (layer "B.Cu") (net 1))
 (segment (start 107.42375 105.368793) (end 107.57125 105.368793) (width 0.25) (layer "B.Cu") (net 1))
 (segment (start 138.552738 105.491531) (end 139.695 106.633793) (width 0.25) (layer "B.Cu") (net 1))
 (segment (start 127.4 82.293793) (end 111.45 82.293793) (width 0.25) (layer "B.Cu") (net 1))
 (segment (start 154.1875 82.293793) (end 153.8 82.293793) (width 0.25) (layer "B.Cu") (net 1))
 (segment (start 137.46375 105.268793) (end 137.30625 105.268793) (width 0.25) (layer "B.Cu") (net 1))
 (segment (start 104.135 107.528283) (end 104.135 111.579829) (width 0.25) (layer "B.Cu") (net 1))
 (segment (start 128.5625 82.293793) (end 153.025 82.293793) (width 0.25) (layer "B.Cu") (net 1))
 (segment (start 132.153125 105.268793) (end 132.321875 105.268793) (width 0.25) (layer "B.Cu") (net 1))
 (segment (start 132.659375 105.268793) (end 132.490625 105.268793) (width 0.25) (layer "B.Cu") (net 1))
 (arc (start 133.488648 105.507441) (mid 133.224309 105.330815) (end 132.9125 105.268793) (width 0.25) (layer "B.Cu") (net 1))
 (arc (start 113.05 107.672041) (mid 113.173448 108.292658) (end 113.525 108.818793) (width 0.25) (layer "B.Cu") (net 1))
 (arc (start 147.315 104.731054) (mid 147.274067 104.936837) (end 147.1575 105.111293) (width 0.25) (layer "B.Cu") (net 1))
 (arc (start 138.552738 105.491531) (mid 138.306021 105.32668) (end 138.015 105.268793) (width 0.25) (layer "B.Cu") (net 1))
 (arc (start 120.438352 109.293793) (mid 121.00344 109.181389) (end 121.4825 108.861293) (width 0.25) (layer "B.Cu") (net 1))
 (arc (start 104.135 107.528283) (mid 104.299381 106.701881) (end 104.7675 106.001293) (width 0.25) (layer "B.Cu") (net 1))
 (arc (start 122.282499 105.636292) (mid 122.689561 105.364302) (end 123.169723 105.268793) (width 0.25) (layer "B.Cu") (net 1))
 (arc (start 146.777261 105.268793) (mid 146.983044 105.22786) (end 147.1575 105.111293) (width 0.25) (layer "B.Cu") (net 1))
 (arc (start 106.39519 82.523602) (mid 106.649739 82.353518) (end 106.95 82.293793) (width 0.25) (layer "B.Cu") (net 1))
 (arc (start 96.696036 119.018793) (mid 98.778426 118.604579) (end 100.543792 117.425) (width 0.25) (layer "B.Cu") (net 1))
 (arc (start 80.0235 83.020293) (mid 79.485811 83.825001) (end 79.297 84.774219) (width 0.25) (layer "B.Cu") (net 1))
 (arc (start 128.664055 104.964737) (mid 128.327267 105.189771) (end 127.93 105.268793) (width 0.25) (layer "B.Cu") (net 1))
 (arc (start 155.497 83.867745) (mid 155.37719 83.265419) (end 155.036 82.754793) (width 0.25) (layer "B.Cu") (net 1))
 (arc (start 114.671751 109.293793) (mid 114.051133 109.170344) (end 113.525 108.818793) (width 0.25) (layer "B.Cu") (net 1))
 (arc (start 128.5625 82.293793) (mid 128.920503 82.365004) (end 129.224003 82.567796) (width 0.25) (layer "B.Cu") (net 1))
 (arc (start 80.0235 83.020293) (mid 80.828208 82.482604) (end 81.777426 82.293793) (width 0.25) (layer "B.Cu") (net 1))
 (arc (start 129.5235 82.867293) (mid 129.947952 83.50253) (end 130.097 84.251844) (width 0.25) (layer "B.Cu") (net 1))
 (arc (start 112.6875 105.731293) (mid 112.285976 105.463003) (end 111.812347 105.368793) (width 0.25) (layer "B.Cu") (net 1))
 (arc (start 180.311 82.879793) (mid 179.661916 82.446089) (end 178.89627 82.293793) (width 0.25) (layer "B.Cu") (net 1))
 (arc (start 104.697 85.305293) (mid 104.896115 84.304269) (end 105.46315 83.455642) (width 0.25) (layer "B.Cu") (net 1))
 (arc (start 102.541207 115.427585) (mid 103.720786 113.662219) (end 104.135 111.579829) (width 0.25) (layer "B.Cu") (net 1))
 (arc (start 113.05 106.47563) (mid 112.979829 106.122858) (end 112.78 105.823793) (width 0.25) (layer "B.Cu") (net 1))
 (arc (start 121.915 106.318793) (mid 121.972887 106.02777) (end 122.137738 105.781054) (width 0.25) (layer "B.Cu") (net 1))
 (arc (start 113.05 106.47563) (mid 113.147636 106.329507) (end 113.32 106.363793) (width 0.25) (layer "B.Cu") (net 1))
 (arc (start 106.29449 105.368793) (mid 105.468088 105.533174) (end 104.7675 106.001293) (width 0.25) (layer "B.Cu") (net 1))
 (arc (start 121.915 107.817145) (mid 121.802596 108.382233) (end 121.4825 108.861293) (width 0.25) (layer "B.Cu") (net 1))
 (arc (start 180.311 82.879793) (mid 180.744703 83.528876) (end 180.897 84.294522) (width 0.25) (layer "B.Cu") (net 1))
 (arc (start 108.148596 105.160196) (mid 107.917544 105.31458) (end 107.645 105.368793) (width 0.25) (layer "B.Cu") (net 1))
 (arc (start 154.849003 82.567796) (mid 154.545503 82.365004) (end 154.1875 82.293793) (width 0.25) (layer "B.Cu") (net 1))
 (arc (start 113.9425 106.633793) (mid 113.616832 106.569013) (end 113.340744 106.384537) (width 0.25) (layer "B.Cu") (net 1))
 (segment (start 103.605 102.198793) (end 103.652399 102.246192) (width 0.25) (layer "F.Cu") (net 4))
 (segment (start 86.945799 101.668793) (end 102.325466 101.668793) (width 0.25) (layer "F.Cu") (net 4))
 (segment (start 82.55 106.064592) (end 82.55 111.398793) (width 0.25) (layer "F.Cu") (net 4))
 (segment (start 104.135 103.411293) (end 104.135 104.093793) (width 0.25) (layer "F.Cu") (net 4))
 (arc (start 86.945799 101.668793) (mid 85.263599 102.003403) (end 83.8375 102.956293) (width 0.25) (layer "F.Cu") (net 4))
 (arc (start 104.135 103.411293) (mid 104.009576 102.780745) (end 103.652399 102.246192) (width 0.25) (layer "F.Cu") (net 4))
 (arc (start 103.605 102.198793) (mid 103.017944 101.806535) (end 102.325466 101.668793) (width 0.25) (layer "F.Cu") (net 4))
 (arc (start 83.8375 102.956293) (mid 82.88461 104.382392) (end 82.55 106.064592) (width 0.25) (layer "F.Cu") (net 4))
 (segment (start 85.125 112.581643) (end 85.125 107.368146) (width 0.25) (layer "F.Cu") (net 3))
 (segment (start 101.5975 102.516293) (end 101.4 102.318793) (width 0.25) (layer "F.Cu") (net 3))
 (segment (start 101.595 102.527328) (end 101.595 104.093793) (width 0.25) (layer "F.Cu") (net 3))
 (segment (start 83.76785 113.938793) (end 82.55 113.938793) (width 0.25) (layer "F.Cu") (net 3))
 (segment (start 90.374353 102.118793) (end 100.917157 102.118793) (width 0.25) (layer "F.Cu") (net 3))
 (arc (start 86.6625 103.656293) (mid 88.365512 102.518376) (end 90.374353 102.118793) (width 0.25) (layer "F.Cu") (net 3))
 (arc (start 101.4 102.318793) (mid 101.178469 102.170771) (end 100.917157 102.118793) (width 0.25) (layer "F.Cu") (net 3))
 (arc (start 83.76785 113.938793) (mid 84.287208 113.835486) (end 84.7275 113.541293) (width 0.25) (layer "F.Cu") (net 3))
 (arc (start 85.125 112.581643) (mid 85.021693 113.101001) (end 84.7275 113.541293) (width 0.25) (layer "F.Cu") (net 3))
 (arc (start 101.5975 102.521293) (mid 101.595649 102.524061) (end 101.595 102.527328) (width 0.25) (layer "F.Cu") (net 3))
 (arc (start 85.125 107.368146) (mid 85.524583 105.359305) (end 86.6625 103.656293) (width 0.25) (layer "F.Cu") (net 3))
 (arc (start 101.5975 102.516293) (mid 101.598535 102.518793) (end 101.5975 102.521293) (width 0.25) (layer "F.Cu") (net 3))
 (segment (start 116.835 101.520673) (end 116.835 104.093793) (width 0.25) (layer "B.Cu") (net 15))
 (segment (start 117.17 100.711912) (end 117.17 88.928793) (width 0.25) (layer "B.Cu") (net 15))
 (arc (start 117.0025 101.116293) (mid 117.126468 100.930761) (end 117.17 100.711912) (width 0.25) (layer "B.Cu") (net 15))
 (arc (start 117.0025 101.116293) (mid 116.878531 101.301824) (end 116.835 101.520673) (width 0.25) (layer "B.Cu") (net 15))
 (segment (start 160.221036 102.193793) (end 122.314429 102.193793) (width 0.25) (layer "B.Cu") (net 5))
 (segment (start 166.376207 98.292585) (end 164.068792 100.6) (width 0.25) (layer "B.Cu") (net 5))
 (segment (start 120.65 103.858222) (end 120.65 104.457231) (width 0.25) (layer "B.Cu") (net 5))
 (segment (start 167.97 94.444829) (end 167.97 88.928793) (width 0.25) (layer "B.Cu") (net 5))
 (segment (start 120.0125 105.996293) (end 119.375 106.633793) (width 0.25) (layer "B.Cu") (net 5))
 (arc (start 160.221036 102.193793) (mid 162.303426 101.779579) (end 164.068792 100.6) (width 0.25) (layer "B.Cu") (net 5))
 (arc (start 121.1375 102.681293) (mid 121.677479 102.32049) (end 122.314429 102.193793) (width 0.25) (layer "B.Cu") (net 5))
 (arc (start 167.97 94.444829) (mid 167.555786 96.527219) (end 166.376207 98.292585) (width 0.25) (layer "B.Cu") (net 5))
 (arc (start 120.0125 105.996293) (mid 120.484319 105.290165) (end 120.65 104.457231) (width 0.25) (layer "B.Cu") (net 5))
 (arc (start 120.65 103.858222) (mid 120.776697 103.221272) (end 121.1375 102.681293) (width 0.25) (layer "B.Cu") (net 5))
 (segment (start 137.54257 101.293793) (end 120.617982 101.293793) (width 0.25) (layer "B.Cu") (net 7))
 (segment (start 118.1 104.474302) (end 118.1 103.811775) (width 0.25) (layer "B.Cu") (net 7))
 (segment (start 142.57 96.266363) (end 142.57 88.928793) (width 0.25) (layer "B.Cu") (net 7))
 (segment (start 117.4675 106.001293) (end 116.835 106.633793) (width 0.25) (layer "B.Cu") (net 7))
 (arc (start 137.54257 101.293793) (mid 139.466484 100.911102) (end 141.0975 99.821293) (width 0.25) (layer "B.Cu") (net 7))
 (arc (start 117.4675 106.001293) (mid 117.935618 105.300703) (end 118.1 104.474302) (width 0.25) (layer "B.Cu") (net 7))
 (arc (start 118.8375 102.031293) (mid 119.654392 101.485463) (end 120.617982 101.293793) (width 0.25) (layer "B.Cu") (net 7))
 (arc (start 118.8375 102.031293) (mid 118.29167 102.848185) (end 118.1 103.811775) (width 0.25) (layer "B.Cu") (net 7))
 (arc (start 142.57 96.266363) (mid 142.187309 98.190277) (end 141.0975 99.821293) (width 0.25) (layer "B.Cu") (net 7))
 (segment (start 110.7222 101.568793) (end 72.253963 101.568793) (width 0.25) (layer "B.Cu") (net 6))
 (segment (start 68.406207 99.975) (end 67.963792 99.532585) (width 0.25) (layer "B.Cu") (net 6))
 (segment (start 111.755 102.601592) (end 111.755 104.093793) (width 0.25) (layer "B.Cu") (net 6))
 (segment (start 66.37 95.684829) (end 66.37 88.928793) (width 0.25) (layer "B.Cu") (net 6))
 (arc (start 67.963792 99.532585) (mid 66.784213 97.767219) (end 66.37 95.684829) (width 0.25) (layer "B.Cu") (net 6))
 (arc (start 68.406207 99.975) (mid 70.171572 101.154579) (end 72.253963 101.568793) (width 0.25) (layer "B.Cu") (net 6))
 (arc (start 110.7222 101.568793) (mid 111.117435 101.64741) (end 111.4525 101.871293) (width 0.25) (layer "B.Cu") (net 6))
 (arc (start 111.755 102.601592) (mid 111.676382 102.206357) (end 111.4525 101.871293) (width 0.25) (layer "B.Cu") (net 6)))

